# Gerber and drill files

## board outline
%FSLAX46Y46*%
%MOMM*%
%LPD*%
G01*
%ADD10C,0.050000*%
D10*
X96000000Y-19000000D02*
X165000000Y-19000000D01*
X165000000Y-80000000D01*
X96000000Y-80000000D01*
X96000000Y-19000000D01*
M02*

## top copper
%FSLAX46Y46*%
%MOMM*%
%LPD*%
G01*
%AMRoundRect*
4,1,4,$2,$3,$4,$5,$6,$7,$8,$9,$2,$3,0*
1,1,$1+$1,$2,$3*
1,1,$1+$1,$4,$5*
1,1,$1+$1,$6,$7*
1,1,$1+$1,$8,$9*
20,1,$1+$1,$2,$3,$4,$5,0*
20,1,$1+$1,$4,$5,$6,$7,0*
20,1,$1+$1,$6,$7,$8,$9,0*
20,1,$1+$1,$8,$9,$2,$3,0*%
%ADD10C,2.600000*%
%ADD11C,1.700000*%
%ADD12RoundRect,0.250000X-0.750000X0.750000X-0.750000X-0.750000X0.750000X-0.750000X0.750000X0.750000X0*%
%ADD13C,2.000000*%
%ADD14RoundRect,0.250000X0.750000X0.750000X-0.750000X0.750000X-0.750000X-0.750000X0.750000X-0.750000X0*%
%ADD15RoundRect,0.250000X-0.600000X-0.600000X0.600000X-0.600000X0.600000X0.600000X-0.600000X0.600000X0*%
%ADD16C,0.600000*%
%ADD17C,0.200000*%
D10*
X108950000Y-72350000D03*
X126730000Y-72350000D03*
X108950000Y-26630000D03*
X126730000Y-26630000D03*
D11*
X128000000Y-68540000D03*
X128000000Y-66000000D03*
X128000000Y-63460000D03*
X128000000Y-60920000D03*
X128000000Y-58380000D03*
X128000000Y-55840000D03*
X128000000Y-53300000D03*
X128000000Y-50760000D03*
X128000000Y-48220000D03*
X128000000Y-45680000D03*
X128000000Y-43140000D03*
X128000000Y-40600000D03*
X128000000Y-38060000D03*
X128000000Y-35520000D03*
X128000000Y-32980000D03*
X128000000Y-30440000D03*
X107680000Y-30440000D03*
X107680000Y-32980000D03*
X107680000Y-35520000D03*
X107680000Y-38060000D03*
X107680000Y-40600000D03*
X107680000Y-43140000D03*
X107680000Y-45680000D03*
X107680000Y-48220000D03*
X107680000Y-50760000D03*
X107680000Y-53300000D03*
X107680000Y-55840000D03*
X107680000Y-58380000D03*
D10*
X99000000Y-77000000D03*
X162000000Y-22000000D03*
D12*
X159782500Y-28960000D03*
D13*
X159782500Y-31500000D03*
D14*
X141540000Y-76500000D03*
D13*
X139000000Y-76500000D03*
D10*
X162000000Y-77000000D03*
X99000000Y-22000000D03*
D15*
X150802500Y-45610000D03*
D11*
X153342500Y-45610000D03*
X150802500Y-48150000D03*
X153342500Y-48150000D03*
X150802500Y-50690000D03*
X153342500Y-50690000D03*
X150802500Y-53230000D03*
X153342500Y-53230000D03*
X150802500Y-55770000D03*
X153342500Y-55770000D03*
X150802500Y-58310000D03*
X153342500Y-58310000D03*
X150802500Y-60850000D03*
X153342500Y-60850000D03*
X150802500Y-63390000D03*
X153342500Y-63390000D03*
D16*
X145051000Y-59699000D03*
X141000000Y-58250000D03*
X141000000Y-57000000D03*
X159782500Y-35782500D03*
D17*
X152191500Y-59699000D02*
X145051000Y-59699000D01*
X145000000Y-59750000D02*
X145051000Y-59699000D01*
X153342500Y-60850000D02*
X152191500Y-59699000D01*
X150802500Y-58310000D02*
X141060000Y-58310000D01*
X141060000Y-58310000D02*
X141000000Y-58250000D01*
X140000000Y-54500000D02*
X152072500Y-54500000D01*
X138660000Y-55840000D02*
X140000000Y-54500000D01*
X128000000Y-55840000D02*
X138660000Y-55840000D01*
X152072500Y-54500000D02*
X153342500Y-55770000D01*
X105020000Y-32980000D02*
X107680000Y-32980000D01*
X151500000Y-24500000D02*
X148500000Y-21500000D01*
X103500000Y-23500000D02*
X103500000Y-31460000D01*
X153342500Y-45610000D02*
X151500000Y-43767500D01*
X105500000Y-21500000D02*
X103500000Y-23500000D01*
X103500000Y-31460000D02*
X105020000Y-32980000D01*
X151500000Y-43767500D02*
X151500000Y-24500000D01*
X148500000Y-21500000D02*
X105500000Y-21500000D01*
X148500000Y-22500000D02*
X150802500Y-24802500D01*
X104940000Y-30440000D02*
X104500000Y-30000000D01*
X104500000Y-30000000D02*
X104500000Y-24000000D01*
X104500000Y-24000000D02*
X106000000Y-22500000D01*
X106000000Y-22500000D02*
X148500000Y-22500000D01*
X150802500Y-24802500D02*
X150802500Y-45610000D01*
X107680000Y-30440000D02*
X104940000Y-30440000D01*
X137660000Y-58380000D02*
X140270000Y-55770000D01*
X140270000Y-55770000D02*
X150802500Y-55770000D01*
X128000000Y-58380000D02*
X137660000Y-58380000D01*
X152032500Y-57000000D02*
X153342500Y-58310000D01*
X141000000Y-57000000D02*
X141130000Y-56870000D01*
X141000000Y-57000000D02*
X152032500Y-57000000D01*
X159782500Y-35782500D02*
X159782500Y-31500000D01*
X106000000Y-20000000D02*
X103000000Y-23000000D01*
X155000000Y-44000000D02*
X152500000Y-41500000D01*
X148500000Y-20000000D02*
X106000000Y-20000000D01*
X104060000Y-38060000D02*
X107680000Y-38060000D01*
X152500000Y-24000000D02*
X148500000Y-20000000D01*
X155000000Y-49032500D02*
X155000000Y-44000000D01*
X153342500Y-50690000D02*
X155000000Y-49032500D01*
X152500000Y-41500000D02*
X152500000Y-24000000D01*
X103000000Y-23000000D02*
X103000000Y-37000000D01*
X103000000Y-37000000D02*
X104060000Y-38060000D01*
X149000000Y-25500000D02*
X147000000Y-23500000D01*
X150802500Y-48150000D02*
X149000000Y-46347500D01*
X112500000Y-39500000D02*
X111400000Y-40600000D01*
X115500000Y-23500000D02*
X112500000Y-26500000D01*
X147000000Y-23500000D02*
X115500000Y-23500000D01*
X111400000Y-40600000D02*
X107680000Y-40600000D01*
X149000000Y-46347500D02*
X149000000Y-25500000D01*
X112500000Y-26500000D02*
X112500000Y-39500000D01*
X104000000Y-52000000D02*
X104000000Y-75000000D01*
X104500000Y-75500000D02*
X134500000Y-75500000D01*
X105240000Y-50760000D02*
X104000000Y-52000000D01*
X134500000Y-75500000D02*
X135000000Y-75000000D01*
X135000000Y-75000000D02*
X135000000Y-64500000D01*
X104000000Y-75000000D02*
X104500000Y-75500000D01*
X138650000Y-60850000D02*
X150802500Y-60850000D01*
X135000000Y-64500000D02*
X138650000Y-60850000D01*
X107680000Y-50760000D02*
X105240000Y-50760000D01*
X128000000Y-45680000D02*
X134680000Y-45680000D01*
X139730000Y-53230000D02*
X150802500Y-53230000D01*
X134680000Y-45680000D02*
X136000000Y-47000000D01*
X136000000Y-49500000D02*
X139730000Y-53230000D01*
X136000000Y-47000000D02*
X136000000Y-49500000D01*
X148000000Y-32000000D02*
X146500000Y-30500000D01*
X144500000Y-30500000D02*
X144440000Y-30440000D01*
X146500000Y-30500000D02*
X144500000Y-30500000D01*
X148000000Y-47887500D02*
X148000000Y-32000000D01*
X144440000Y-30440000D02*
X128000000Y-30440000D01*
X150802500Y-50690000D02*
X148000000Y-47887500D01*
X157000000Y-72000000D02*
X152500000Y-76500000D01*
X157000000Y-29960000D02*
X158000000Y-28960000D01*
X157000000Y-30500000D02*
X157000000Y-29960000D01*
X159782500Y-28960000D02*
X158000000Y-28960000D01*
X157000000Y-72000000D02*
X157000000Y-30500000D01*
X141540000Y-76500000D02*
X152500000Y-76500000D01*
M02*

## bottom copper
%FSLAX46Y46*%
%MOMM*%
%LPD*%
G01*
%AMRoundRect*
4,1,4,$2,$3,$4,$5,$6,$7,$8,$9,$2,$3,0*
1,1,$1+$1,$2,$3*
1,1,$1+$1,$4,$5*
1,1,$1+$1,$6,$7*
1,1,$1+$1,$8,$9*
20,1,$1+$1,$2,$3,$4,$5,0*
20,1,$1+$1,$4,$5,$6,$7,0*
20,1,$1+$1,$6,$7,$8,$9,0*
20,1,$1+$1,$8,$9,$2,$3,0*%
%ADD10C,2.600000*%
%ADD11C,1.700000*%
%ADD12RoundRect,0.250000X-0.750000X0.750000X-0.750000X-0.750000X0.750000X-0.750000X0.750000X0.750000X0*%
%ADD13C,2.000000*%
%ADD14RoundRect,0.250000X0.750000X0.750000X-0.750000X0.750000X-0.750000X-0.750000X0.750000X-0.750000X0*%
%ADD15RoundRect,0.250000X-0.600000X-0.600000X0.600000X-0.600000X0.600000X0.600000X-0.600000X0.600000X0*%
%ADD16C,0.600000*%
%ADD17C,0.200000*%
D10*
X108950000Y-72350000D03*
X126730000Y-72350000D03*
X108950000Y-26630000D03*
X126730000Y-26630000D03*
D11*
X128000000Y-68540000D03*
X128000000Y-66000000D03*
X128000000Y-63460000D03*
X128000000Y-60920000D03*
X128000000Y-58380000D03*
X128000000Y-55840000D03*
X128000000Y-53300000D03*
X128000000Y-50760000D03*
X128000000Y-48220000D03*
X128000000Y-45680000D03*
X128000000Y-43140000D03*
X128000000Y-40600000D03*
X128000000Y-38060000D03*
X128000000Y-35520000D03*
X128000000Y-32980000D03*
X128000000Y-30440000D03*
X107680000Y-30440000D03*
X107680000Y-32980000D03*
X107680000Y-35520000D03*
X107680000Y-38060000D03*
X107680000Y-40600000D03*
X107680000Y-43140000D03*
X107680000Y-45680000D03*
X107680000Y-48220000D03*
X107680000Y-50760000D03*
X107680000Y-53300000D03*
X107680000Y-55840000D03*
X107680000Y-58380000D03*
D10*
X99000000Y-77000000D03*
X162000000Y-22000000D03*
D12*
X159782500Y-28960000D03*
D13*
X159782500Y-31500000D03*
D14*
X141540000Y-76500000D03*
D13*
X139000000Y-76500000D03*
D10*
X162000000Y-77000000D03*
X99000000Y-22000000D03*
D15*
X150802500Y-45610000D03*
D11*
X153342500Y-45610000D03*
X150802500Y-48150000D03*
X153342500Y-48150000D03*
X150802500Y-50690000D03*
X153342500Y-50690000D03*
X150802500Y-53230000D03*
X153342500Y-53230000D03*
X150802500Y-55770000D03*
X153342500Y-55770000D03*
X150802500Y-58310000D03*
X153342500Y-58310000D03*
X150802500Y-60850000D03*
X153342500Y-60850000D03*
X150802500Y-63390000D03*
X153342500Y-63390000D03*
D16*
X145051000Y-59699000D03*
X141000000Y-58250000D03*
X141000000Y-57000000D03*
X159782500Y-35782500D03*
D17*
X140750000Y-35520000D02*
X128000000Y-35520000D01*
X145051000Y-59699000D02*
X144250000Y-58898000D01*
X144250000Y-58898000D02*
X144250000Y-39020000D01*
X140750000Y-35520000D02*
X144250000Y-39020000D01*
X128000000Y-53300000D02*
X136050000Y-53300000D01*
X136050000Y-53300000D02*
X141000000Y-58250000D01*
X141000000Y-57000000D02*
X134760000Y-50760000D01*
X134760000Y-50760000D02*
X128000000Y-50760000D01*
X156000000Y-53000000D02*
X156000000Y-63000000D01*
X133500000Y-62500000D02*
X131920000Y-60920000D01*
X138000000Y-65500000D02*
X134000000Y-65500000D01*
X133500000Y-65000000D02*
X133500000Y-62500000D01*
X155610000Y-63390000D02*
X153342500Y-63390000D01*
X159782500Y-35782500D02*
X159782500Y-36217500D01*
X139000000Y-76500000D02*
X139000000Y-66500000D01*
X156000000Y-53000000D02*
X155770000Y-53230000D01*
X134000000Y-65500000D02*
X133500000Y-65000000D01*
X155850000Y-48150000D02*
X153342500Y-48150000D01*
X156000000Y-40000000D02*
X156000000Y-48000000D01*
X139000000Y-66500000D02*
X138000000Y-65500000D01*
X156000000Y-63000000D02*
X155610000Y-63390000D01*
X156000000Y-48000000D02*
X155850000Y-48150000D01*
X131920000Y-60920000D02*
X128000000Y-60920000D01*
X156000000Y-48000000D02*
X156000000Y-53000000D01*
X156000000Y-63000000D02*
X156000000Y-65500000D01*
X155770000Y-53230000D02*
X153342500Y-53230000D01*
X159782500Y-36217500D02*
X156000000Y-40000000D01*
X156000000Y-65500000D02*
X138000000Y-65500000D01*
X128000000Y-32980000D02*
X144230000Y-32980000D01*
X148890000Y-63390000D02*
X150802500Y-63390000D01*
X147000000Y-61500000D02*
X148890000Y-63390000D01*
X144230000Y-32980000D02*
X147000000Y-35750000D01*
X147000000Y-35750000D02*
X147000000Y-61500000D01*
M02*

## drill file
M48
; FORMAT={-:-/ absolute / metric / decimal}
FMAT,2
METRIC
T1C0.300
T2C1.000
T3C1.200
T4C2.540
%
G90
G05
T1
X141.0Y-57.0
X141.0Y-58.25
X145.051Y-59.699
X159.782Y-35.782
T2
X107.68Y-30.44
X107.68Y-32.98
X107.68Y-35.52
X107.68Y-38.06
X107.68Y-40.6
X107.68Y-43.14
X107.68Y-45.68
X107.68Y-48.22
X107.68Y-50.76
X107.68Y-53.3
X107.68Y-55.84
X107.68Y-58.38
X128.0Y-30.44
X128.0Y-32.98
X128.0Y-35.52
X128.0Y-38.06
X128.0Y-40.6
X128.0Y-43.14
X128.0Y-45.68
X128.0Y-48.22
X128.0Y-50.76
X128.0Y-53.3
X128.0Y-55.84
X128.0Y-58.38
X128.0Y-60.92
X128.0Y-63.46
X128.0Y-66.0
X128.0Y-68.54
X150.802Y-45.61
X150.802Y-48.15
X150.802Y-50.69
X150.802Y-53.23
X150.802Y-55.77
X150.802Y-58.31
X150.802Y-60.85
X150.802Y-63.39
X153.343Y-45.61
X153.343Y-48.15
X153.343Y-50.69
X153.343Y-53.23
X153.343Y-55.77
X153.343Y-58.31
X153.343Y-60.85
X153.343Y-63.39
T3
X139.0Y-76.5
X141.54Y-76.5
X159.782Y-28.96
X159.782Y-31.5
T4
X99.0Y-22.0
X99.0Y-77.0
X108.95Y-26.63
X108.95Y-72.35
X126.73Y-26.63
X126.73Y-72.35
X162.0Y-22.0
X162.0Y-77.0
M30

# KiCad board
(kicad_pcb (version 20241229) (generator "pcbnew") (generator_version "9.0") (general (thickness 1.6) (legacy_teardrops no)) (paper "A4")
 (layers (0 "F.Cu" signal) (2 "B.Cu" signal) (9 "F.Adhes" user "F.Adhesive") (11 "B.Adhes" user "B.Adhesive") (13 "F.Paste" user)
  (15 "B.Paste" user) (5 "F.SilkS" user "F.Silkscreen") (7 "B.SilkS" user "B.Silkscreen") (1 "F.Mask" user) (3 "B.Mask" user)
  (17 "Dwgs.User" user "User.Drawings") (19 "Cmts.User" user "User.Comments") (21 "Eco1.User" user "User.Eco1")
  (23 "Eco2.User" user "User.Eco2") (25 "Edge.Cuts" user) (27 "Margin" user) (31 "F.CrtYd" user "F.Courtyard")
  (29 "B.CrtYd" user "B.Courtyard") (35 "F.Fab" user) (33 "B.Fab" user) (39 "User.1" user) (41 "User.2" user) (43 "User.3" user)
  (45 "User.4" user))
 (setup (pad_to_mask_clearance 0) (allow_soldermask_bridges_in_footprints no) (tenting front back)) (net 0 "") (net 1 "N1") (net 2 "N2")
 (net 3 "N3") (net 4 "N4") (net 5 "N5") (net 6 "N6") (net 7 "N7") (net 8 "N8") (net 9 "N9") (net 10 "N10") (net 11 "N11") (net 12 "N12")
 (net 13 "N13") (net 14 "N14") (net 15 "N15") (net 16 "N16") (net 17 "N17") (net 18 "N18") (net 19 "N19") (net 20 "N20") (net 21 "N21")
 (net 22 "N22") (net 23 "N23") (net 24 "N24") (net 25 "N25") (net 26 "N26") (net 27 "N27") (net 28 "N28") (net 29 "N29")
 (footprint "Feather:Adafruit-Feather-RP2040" (layer "F.Cu") (at 117.84 49.49 90)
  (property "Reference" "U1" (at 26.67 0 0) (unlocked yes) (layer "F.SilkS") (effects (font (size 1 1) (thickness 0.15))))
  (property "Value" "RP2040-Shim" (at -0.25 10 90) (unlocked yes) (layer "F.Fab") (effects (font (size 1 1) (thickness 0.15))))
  (pad "" np_thru_hole circle (at -22.86 -8.89 90) (size 2.6 2.6) (drill 2.54) (layers "*.Cu" "*.Mask") (solder_mask_margin 1.3)
   (clearance 1.3))
  (pad "" np_thru_hole circle (at -22.86 8.89 90) (size 2.6 2.6) (drill 2.54) (layers "*.Cu" "*.Mask") (solder_mask_margin 1.3)
   (clearance 1.3))
  (pad "" np_thru_hole circle (at 22.86 -8.89 90) (size 2.6 2.6) (drill 2.54) (layers "*.Cu" "*.Mask") (solder_mask_margin 1.3)
   (clearance 1.3))
  (pad "" np_thru_hole circle (at 22.86 8.89 90) (size 2.6 2.6) (drill 2.54) (layers "*.Cu" "*.Mask") (solder_mask_margin 1.3)
   (clearance 1.3))
  (pad "1" thru_hole circle (at -19.05 10.16 90) (size 1.7 1.7) (drill 1) (layers "*.Cu" "*.Mask") (remove_unused_layers no) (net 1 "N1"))
  (pad "2" thru_hole circle (at -16.51 10.16 90) (size 1.7 1.7) (drill 1) (layers "*.Cu" "*.Mask") (remove_unused_layers no) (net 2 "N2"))
  (pad "3" thru_hole circle (at -13.97 10.16 90) (size 1.7 1.7) (drill 1) (layers "*.Cu" "*.Mask") (remove_unused_layers no) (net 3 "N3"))
  (pad "4" thru_hole circle (at -11.43 10.16 90) (size 1.7 1.7) (drill 1) (layers "*.Cu" "*.Mask") (remove_unused_layers no) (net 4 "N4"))
  (pad "5" thru_hole circle (at -8.89 10.16 90) (size 1.7 1.7) (drill 1) (layers "*.Cu" "*.Mask") (remove_unused_layers no) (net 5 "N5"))
  (pad "6" thru_hole circle (at -6.35 10.16 90) (size 1.7 1.7) (drill 1) (layers "*.Cu" "*.Mask") (remove_unused_layers no) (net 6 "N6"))
  (pad "7" thru_hole circle (at -3.81 10.16 90) (size 1.7 1.7) (drill 1) (layers "*.Cu" "*.Mask") (remove_unused_layers no) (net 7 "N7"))
  (pad "8" thru_hole circle (at -1.27 10.16 90) (size 1.7 1.7) (drill 1) (layers "*.Cu" "*.Mask") (remove_unused_layers no) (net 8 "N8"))
  (pad "9" thru_hole circle (at 1.27 10.16 90) (size 1.7 1.7) (drill 1) (layers "*.Cu" "*.Mask") (remove_unused_layers no) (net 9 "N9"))
  (pad "10" thru_hole circle (at 3.81 10.16 90) (size 1.7 1.7) (drill 1) (layers "*.Cu" "*.Mask") (remove_unused_layers no) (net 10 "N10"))
  (pad "11" thru_hole circle (at 6.35 10.16 90) (size 1.7 1.7) (drill 1) (layers "*.Cu" "*.Mask") (remove_unused_layers no) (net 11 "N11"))
  (pad "12" thru_hole circle (at 8.89 10.16 90) (size 1.7 1.7) (drill 1) (layers "*.Cu" "*.Mask") (remove_unused_layers no) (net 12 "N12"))
  (pad "13" thru_hole circle (at 11.43 10.16 90) (size 1.7 1.7) (drill 1) (layers "*.Cu" "*.Mask") (remove_unused_layers no) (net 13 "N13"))
  (pad "14" thru_hole circle (at 13.97 10.16 90) (size 1.7 1.7) (drill 1) (layers "*.Cu" "*.Mask") (remove_unused_layers no) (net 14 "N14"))
  (pad "15" thru_hole circle (at 16.51 10.16 90) (size 1.7 1.7) (drill 1) (layers "*.Cu" "*.Mask") (remove_unused_layers no) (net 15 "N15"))
  (pad "16" thru_hole circle (at 19.05 10.16 90) (size 1.7 1.7) (drill 1) (layers "*.Cu" "*.Mask") (remove_unused_layers no) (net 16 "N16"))
  (pad "17" thru_hole circle (at 19.05 -10.16 90) (size 1.7 1.7) (drill 1) (layers "*.Cu" "*.Mask") (remove_unused_layers no) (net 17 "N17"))
  (pad "18" thru_hole circle (at 16.51 -10.16 90) (size 1.7 1.7) (drill 1) (layers "*.Cu" "*.Mask") (remove_unused_layers no) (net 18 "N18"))
  (pad "19" thru_hole circle (at 13.97 -10.16 90) (size 1.7 1.7) (drill 1) (layers "*.Cu" "*.Mask") (remove_unused_layers no) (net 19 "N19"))
  (pad "20" thru_hole circle (at 11.43 -10.16 90) (size 1.7 1.7) (drill 1) (layers "*.Cu" "*.Mask") (remove_unused_layers no) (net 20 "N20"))
  (pad "21" thru_hole circle (at 8.89 -10.16 90) (size 1.7 1.7) (drill 1) (layers "*.Cu" "*.Mask") (remove_unused_layers no) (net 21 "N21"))
  (pad "22" thru_hole circle (at 6.35 -10.16 90) (size 1.7 1.7) (drill 1) (layers "*.Cu" "*.Mask") (remove_unused_layers no) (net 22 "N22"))
  (pad "23" thru_hole circle (at 3.81 -10.16 90) (size 1.7 1.7) (drill 1) (layers "*.Cu" "*.Mask") (remove_unused_layers no) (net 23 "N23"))
  (pad "24" thru_hole circle (at 1.27 -10.16 90) (size 1.7 1.7) (drill 1) (layers "*.Cu" "*.Mask") (remove_unused_layers no) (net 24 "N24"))
  (pad "25" thru_hole circle (at -1.27 -10.16 90) (size 1.7 1.7) (drill 1) (layers "*.Cu" "*.Mask") (remove_unused_layers no) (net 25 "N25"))
  (pad "26" thru_hole circle (at -3.81 -10.16 90) (size 1.7 1.7) (drill 1) (layers "*.Cu" "*.Mask") (remove_unused_layers no) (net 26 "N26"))
  (pad "27" thru_hole circle (at -6.35 -10.16 90) (size 1.7 1.7) (drill 1) (layers "*.Cu" "*.Mask") (remove_unused_layers no) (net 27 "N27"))
  (pad "28" thru_hole circle (at -8.89 -10.16 90) (size 1.7 1.7) (drill 1) (layers "*.Cu" "*.Mask") (remove_unused_layers no) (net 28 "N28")))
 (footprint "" (layer "F.Cu") (at 99 77)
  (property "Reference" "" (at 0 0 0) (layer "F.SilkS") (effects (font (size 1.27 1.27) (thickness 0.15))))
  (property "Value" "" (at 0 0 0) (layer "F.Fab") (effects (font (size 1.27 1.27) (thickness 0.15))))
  (pad "" np_thru_hole circle (at 0 0 90) (size 2.6 2.6) (drill 2.54) (layers "*.Cu" "*.Mask") (solder_mask_margin 1.3) (clearance 1.3)))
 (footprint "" (layer "F.Cu") (at 162 22)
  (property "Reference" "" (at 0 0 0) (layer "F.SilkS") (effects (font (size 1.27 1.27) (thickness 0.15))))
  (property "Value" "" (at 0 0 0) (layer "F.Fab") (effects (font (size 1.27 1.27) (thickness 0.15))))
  (pad "" np_thru_hole circle (at 0 0 90) (size 2.6 2.6) (drill 2.54) (layers "*.Cu" "*.Mask") (solder_mask_margin 1.3) (clearance 1.3)))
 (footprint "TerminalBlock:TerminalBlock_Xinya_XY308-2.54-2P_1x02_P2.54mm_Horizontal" (layer "F.Cu") (at 159.7825 28.96 -90)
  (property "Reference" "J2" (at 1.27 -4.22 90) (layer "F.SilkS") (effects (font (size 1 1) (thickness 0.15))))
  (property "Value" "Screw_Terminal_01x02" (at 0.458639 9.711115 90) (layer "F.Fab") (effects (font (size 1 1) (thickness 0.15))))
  (pad "1" thru_hole roundrect (at 0 0 270) (size 2 2) (drill 1.2) (layers "*.Cu" "*.Mask") (remove_unused_layers no)
   (roundrect_rratio 0.125) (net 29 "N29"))
  (pad "2" thru_hole circle (at 2.54 0 270) (size 2 2) (drill 1.2) (layers "*.Cu" "*.Mask") (remove_unused_layers no) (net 4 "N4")))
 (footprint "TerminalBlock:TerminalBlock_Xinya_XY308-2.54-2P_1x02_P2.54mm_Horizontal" (layer "F.Cu") (at 141.54 76.5 180)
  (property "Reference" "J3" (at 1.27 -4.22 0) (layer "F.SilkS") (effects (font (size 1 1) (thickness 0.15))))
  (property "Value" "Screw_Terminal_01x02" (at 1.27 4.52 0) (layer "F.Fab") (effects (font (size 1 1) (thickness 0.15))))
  (pad "1" thru_hole roundrect (at 0 0 180) (size 2 2) (drill 1.2) (layers "*.Cu" "*.Mask") (remove_unused_layers no)
   (roundrect_rratio 0.125) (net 29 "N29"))
  (pad "2" thru_hole circle (at 2.54 0 180) (size 2 2) (drill 1.2) (layers "*.Cu" "*.Mask") (remove_unused_layers no) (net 4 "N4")))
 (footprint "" (layer "F.Cu") (at 162 77)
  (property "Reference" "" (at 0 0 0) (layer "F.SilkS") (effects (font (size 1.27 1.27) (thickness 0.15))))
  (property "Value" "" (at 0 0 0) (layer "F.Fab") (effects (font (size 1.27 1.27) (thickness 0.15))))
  (pad "" np_thru_hole circle (at 0 0 90) (size 2.6 2.6) (drill 2.54) (layers "*.Cu" "*.Mask") (solder_mask_margin 1.3) (clearance 1.3)))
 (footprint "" (layer "F.Cu") (at 99 22)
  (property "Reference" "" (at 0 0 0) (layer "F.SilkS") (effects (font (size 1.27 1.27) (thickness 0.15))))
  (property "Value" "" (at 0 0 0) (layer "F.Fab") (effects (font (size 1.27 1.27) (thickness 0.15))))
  (pad "" np_thru_hole circle (at 0 0 90) (size 2.6 2.6) (drill 2.54) (layers "*.Cu" "*.Mask") (solder_mask_margin 1.3) (clearance 1.3)))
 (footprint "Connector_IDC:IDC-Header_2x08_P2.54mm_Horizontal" (layer "F.Cu") (at 150.8025 45.61)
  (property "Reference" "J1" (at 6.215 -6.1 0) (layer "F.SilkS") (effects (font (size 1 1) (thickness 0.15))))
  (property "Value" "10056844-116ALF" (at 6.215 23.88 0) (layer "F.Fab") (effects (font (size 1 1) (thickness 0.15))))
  (pad "1" thru_hole roundrect (at 0 0) (size 1.7 1.7) (drill 1) (layers "*.Cu" "*.Mask") (remove_unused_layers no)
   (roundrect_rratio 0.147059) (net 17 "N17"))
  (pad "2" thru_hole circle (at 2.54 0) (size 1.7 1.7) (drill 1) (layers "*.Cu" "*.Mask") (remove_unused_layers no) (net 18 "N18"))
  (pad "3" thru_hole circle (at 0 2.54) (size 1.7 1.7) (drill 1) (layers "*.Cu" "*.Mask") (remove_unused_layers no) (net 21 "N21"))
  (pad "4" thru_hole circle (at 2.54 2.54) (size 1.7 1.7) (drill 1) (layers "*.Cu" "*.Mask") (remove_unused_layers no) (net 4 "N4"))
  (pad "5" thru_hole circle (at 0 5.08) (size 1.7 1.7) (drill 1) (layers "*.Cu" "*.Mask") (remove_unused_layers no) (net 16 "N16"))
  (pad "6" thru_hole circle (at 2.54 5.08) (size 1.7 1.7) (drill 1) (layers "*.Cu" "*.Mask") (remove_unused_layers no) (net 20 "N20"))
  (pad "7" thru_hole circle (at 0 7.62) (size 1.7 1.7) (drill 1) (layers "*.Cu" "*.Mask") (remove_unused_layers no) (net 10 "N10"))
  (pad "8" thru_hole circle (at 2.54 7.62) (size 1.7 1.7) (drill 1) (layers "*.Cu" "*.Mask") (remove_unused_layers no) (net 4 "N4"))
  (pad "9" thru_hole circle (at 0 10.16) (size 1.7 1.7) (drill 1) (layers "*.Cu" "*.Mask") (remove_unused_layers no) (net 5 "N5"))
  (pad "10" thru_hole circle (at 2.54 10.16) (size 1.7 1.7) (drill 1) (layers "*.Cu" "*.Mask") (remove_unused_layers no) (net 6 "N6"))
  (pad "11" thru_hole circle (at 0 12.7) (size 1.7 1.7) (drill 1) (layers "*.Cu" "*.Mask") (remove_unused_layers no) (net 7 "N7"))
  (pad "12" thru_hole circle (at 2.54 12.7) (size 1.7 1.7) (drill 1) (layers "*.Cu" "*.Mask") (remove_unused_layers no) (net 8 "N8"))
  (pad "13" thru_hole circle (at 0 15.24) (size 1.7 1.7) (drill 1) (layers "*.Cu" "*.Mask") (remove_unused_layers no) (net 25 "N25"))
  (pad "14" thru_hole circle (at 2.54 15.24) (size 1.7 1.7) (drill 1) (layers "*.Cu" "*.Mask") (remove_unused_layers no) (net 14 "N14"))
  (pad "15" thru_hole circle (at 0 17.78) (size 1.7 1.7) (drill 1) (layers "*.Cu" "*.Mask") (remove_unused_layers no) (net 15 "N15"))
  (pad "16" thru_hole circle (at 2.54 17.78) (size 1.7 1.7) (drill 1) (layers "*.Cu" "*.Mask") (remove_unused_layers no) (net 4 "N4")))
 (gr_rect (start 96 19) (end 165 80) (stroke (width 0.05) (type solid)) (fill no) (layer "Edge.Cuts"))
 (segment (start 152.1915 59.699) (end 145.051 59.699) (width 0.2) (layer "F.Cu") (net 14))
 (segment (start 145 59.75) (end 145.051 59.699) (width 0.2) (layer "F.Cu") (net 14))
 (segment (start 153.3425 60.85) (end 152.1915 59.699) (width 0.2) (layer "F.Cu") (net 14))
 (via (at 145.051 59.699) (size 0.6) (drill 0.3) (layers "F.Cu" "B.Cu") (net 14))
 (segment (start 140.75 35.52) (end 128 35.52) (width 0.2) (layer "B.Cu") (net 14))
 (segment (start 145.051 59.699) (end 144.25 58.898) (width 0.2) (layer "B.Cu") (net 14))
 (segment (start 144.25 58.898) (end 144.25 39.02) (width 0.2) (layer "B.Cu") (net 14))
 (segment (start 140.75 35.52) (end 144.25 39.02) (width 0.2) (layer "B.Cu") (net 14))
 (segment (start 150.8025 58.31) (end 141.06 58.31) (width 0.2) (layer "F.Cu") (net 7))
 (segment (start 141.06 58.31) (end 141 58.25) (width 0.2) (layer "F.Cu") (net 7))
 (via (at 141 58.25) (size 0.6) (drill 0.3) (layers "F.Cu" "B.Cu") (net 7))
 (segment (start 128 53.3) (end 136.05 53.3) (width 0.2) (layer "B.Cu") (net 7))
 (segment (start 136.05 53.3) (end 141 58.25) (width 0.2) (layer "B.Cu") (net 7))
 (segment (start 140 54.5) (end 152.0725 54.5) (width 0.2) (layer "F.Cu") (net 6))
 (segment (start 138.66 55.84) (end 140 54.5) (width 0.2) (layer "F.Cu") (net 6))
 (segment (start 128 55.84) (end 138.66 55.84) (width 0.2) (layer "F.Cu") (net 6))
 (segment (start 152.0725 54.5) (end 153.3425 55.77) (width 0.2) (layer "F.Cu") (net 6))
 (segment (start 105.02 32.98) (end 107.68 32.98) (width 0.2) (layer "F.Cu") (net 18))
 (segment (start 151.5 24.5) (end 148.5 21.5) (width 0.2) (layer "F.Cu") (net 18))
 (segment (start 103.5 23.5) (end 103.5 31.46) (width 0.2) (layer "F.Cu") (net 18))
 (segment (start 153.3425 45.61) (end 151.5 43.7675) (width 0.2) (layer "F.Cu") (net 18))
 (segment (start 105.5 21.5) (end 103.5 23.5) (width 0.2) (layer "F.Cu") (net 18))
 (segment (start 103.5 31.46) (end 105.02 32.98) (width 0.2) (layer "F.Cu") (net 18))
 (segment (start 151.5 43.7675) (end 151.5 24.5) (width 0.2) (layer "F.Cu") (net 18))
 (segment (start 148.5 21.5) (end 105.5 21.5) (width 0.2) (layer "F.Cu") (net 18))
 (segment (start 148.5 22.5) (end 150.8025 24.8025) (width 0.2) (layer "F.Cu") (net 17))
 (segment (start 104.94 30.44) (end 104.5 30) (width 0.2) (layer "F.Cu") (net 17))
 (segment (start 104.5 30) (end 104.5 24) (width 0.2) (layer "F.Cu") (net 17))
 (segment (start 104.5 24) (end 106 22.5) (width 0.2) (layer "F.Cu") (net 17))
 (segment (start 106 22.5) (end 148.5 22.5) (width 0.2) (layer "F.Cu") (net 17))
 (segment (start 150.8025 24.8025) (end 150.8025 45.61) (width 0.2) (layer "F.Cu") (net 17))
 (segment (start 107.68 30.44) (end 104.94 30.44) (width 0.2) (layer "F.Cu") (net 17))
 (segment (start 137.66 58.38) (end 140.27 55.77) (width 0.2) (layer "F.Cu") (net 5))
 (segment (start 140.27 55.77) (end 150.8025 55.77) (width 0.2) (layer "F.Cu") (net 5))
 (segment (start 128 58.38) (end 137.66 58.38) (width 0.2) (layer "F.Cu") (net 5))
 (segment (start 152.0325 57) (end 153.3425 58.31) (width 0.2) (layer "F.Cu") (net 8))
 (segment (start 141 57) (end 141.13 56.87) (width 0.2) (layer "F.Cu") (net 8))
 (segment (start 141 57) (end 152.0325 57) (width 0.2) (layer "F.Cu") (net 8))
 (via (at 141 57) (size 0.6) (drill 0.3) (layers "F.Cu" "B.Cu") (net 8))
 (segment (start 141 57) (end 134.76 50.76) (width 0.2) (layer "B.Cu") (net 8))
 (segment (start 134.76 50.76) (end 128 50.76) (width 0.2) (layer "B.Cu") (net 8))
 (segment (start 159.7825 35.7825) (end 159.7825 31.5) (width 0.2) (layer "F.Cu") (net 4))
 (via (at 159.7825 35.7825) (size 0.6) (drill 0.3) (layers "F.Cu" "B.Cu") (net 4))
 (segment (start 156 53) (end 156 63) (width 0.2) (layer "B.Cu") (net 4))
 (segment (start 133.5 62.5) (end 131.92 60.92) (width 0.2) (layer "B.Cu") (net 4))
 (segment (start 138 65.5) (end 134 65.5) (width 0.2) (layer "B.Cu") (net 4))
 (segment (start 133.5 65) (end 133.5 62.5) (width 0.2) (layer "B.Cu") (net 4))
 (segment (start 155.61 63.39) (end 153.3425 63.39) (width 0.2) (layer "B.Cu") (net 4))
 (segment (start 159.7825 35.7825) (end 159.7825 36.2175) (width 0.2) (layer "B.Cu") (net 4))
 (segment (start 139 76.5) (end 139 66.5) (width 0.2) (layer "B.Cu") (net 4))
 (segment (start 156 53) (end 155.77 53.23) (width 0.2) (layer "B.Cu") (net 4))
 (segment (start 134 65.5) (end 133.5 65) (width 0.2) (layer "B.Cu") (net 4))
 (segment (start 155.85 48.15) (end 153.3425 48.15) (width 0.2) (layer "B.Cu") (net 4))
 (segment (start 156 40) (end 156 48) (width 0.2) (layer "B.Cu") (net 4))
 (segment (start 139 66.5) (end 138 65.5) (width 0.2) (layer "B.Cu") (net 4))
 (segment (start 156 63) (end 155.61 63.39) (width 0.2) (layer "B.Cu") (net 4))
 (segment (start 156 48) (end 155.85 48.15) (width 0.2) (layer "B.Cu") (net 4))
 (segment (start 131.92 60.92) (end 128 60.92) (width 0.2) (layer "B.Cu") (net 4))
 (segment (start 156 48) (end 156 53) (width 0.2) (layer "B.Cu") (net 4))
 (segment (start 156 63) (end 156 65.5) (width 0.2) (layer "B.Cu") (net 4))
 (segment (start 155.77 53.23) (end 153.3425 53.23) (width 0.2) (layer "B.Cu") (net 4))
 (segment (start 159.7825 36.2175) (end 156 40) (width 0.2) (layer "B.Cu") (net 4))
 (segment (start 156 65.5) (end 138 65.5) (width 0.2) (layer "B.Cu") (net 4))
 (segment (start 128 32.98) (end 144.23 32.98) (width 0.2) (layer "B.Cu") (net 15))
 (segment (start 148.89 63.39) (end 150.8025 63.39) (width 0.2) (layer "B.Cu") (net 15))
 (segment (start 147 61.5) (end 148.89 63.39) (width 0.2) (layer "B.Cu") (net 15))
 (segment (start 144.23 32.98) (end 147 35.75) (width 0.2) (layer "B.Cu") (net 15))
 (segment (start 147 35.75) (end 147 61.5) (width 0.2) (layer "B.Cu") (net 15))
 (segment (start 106 20) (end 103 23) (width 0.2) (layer "F.Cu") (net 20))
 (segment (start 155 44) (end 152.5 41.5) (width 0.2) (layer "F.Cu") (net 20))
 (segment (start 148.5 20) (end 106 20) (width 0.2) (layer "F.Cu") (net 20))
 (segment (start 104.06 38.06) (end 107.68 38.06) (width 0.2) (layer "F.Cu") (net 20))
 (segment (start 152.5 24) (end 148.5 20) (width 0.2) (layer "F.Cu") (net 20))
 (segment (start 155 49.0325) (end 155 44) (width 0.2) (layer "F.Cu") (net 20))
 (segment (start 153.3425 50.69) (end 155 49.0325) (width 0.2) (layer "F.Cu") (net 20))
 (segment (start 152.5 41.5) (end 152.5 24) (width 0.2) (layer "F.Cu") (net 20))
 (segment (start 103 23) (end 103 37) (width 0.2) (layer "F.Cu") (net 20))
 (segment (start 103 37) (end 104.06 38.06) (width 0.2) (layer "F.Cu") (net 20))
 (segment (start 149 25.5) (end 147 23.5) (width 0.2) (layer "F.Cu") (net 21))
 (segment (start 150.8025 48.15) (end 149 46.3475) (width 0.2) (layer "F.Cu") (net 21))
 (segment (start 112.5 39.5) (end 111.4 40.6) (width 0.2) (layer "F.Cu") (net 21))
 (segment (start 115.5 23.5) (end 112.5 26.5) (width 0.2) (layer "F.Cu") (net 21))
 (segment (start 147 23.5) (end 115.5 23.5) (width 0.2) (layer "F.Cu") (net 21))
 (segment (start 111.4 40.6) (end 107.68 40.6) (width 0.2) (layer "F.Cu") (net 21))
 (segment (start 149 46.3475) (end 149 25.5) (width 0.2) (layer "F.Cu") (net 21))
 (segment (start 112.5 26.5) (end 112.5 39.5) (width 0.2) (layer "F.Cu") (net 21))
 (segment (start 104 52) (end 104 75) (width 0.2) (layer "F.Cu") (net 25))
 (segment (start 104.5 75.5) (end 134.5 75.5) (width 0.2) (layer "F.Cu") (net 25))
 (segment (start 105.24 50.76) (end 104 52) (width 0.2) (layer "F.Cu") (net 25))
 (segment (start 134.5 75.5) (end 135 75) (width 0.2) (layer "F.Cu") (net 25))
 (segment (start 135 75) (end 135 64.5) (width 0.2) (layer "F.Cu") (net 25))
 (segment (start 104 75) (end 104.5 75.5) (width 0.2) (layer "F.Cu") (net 25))
 (segment (start 138.65 60.85) (end 150.8025 60.85) (width 0.2) (layer "F.Cu") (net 25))
 (segment (start 135 64.5) (end 138.65 60.85) (width 0.2) (layer "F.Cu") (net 25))
 (segment (start 107.68 50.76) (end 105.24 50.76) (width 0.2) (layer "F.Cu") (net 25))
 (segment (start 128 45.68) (end 134.68 45.68) (width 0.2) (layer "F.Cu") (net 10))
 (segment (start 139.73 53.23) (end 150.8025 53.23) (width 0.2) (layer "F.Cu") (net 10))
 (segment (start 134.68 45.68) (end 136 47) (width 0.2) (layer "F.Cu") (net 10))
 (segment (start 136 49.5) (end 139.73 53.23) (width 0.2) (layer "F.Cu") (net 10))
 (segment (start 136 47) (end 136 49.5) (width 0.2) (layer "F.Cu") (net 10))
 (segment (start 148 32) (end 146.5 30.5) (width 0.2) (layer "F.Cu") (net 16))
 (segment (start 144.5 30.5) (end 144.44 30.44) (width 0.2) (layer "F.Cu") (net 16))
 (segment (start 146.5 30.5) (end 144.5 30.5) (width 0.2) (layer "F.Cu") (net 16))
 (segment (start 148 47.8875) (end 148 32) (width 0.2) (layer "F.Cu") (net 16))
 (segment (start 144.44 30.44) (end 128 30.44) (width 0.2) (layer "F.Cu") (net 16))
 (segment (start 150.8025 50.69) (end 148 47.8875) (width 0.2) (layer "F.Cu") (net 16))
 (segment (start 157 72) (end 152.5 76.5) (width 0.2) (layer "F.Cu") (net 29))
 (segment (start 157 29.96) (end 158 28.96) (width 0.2) (layer "F.Cu") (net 29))
 (segment (start 157 30.5) (end 157 29.96) (width 0.2) (layer "F.Cu") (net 29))
 (segment (start 159.7825 28.96) (end 158 28.96) (width 0.2) (layer "F.Cu") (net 29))
 (segment (start 157 72) (end 157 30.5) (width 0.2) (layer "F.Cu") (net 29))
 (segment (start 141.54 76.5) (end 152.5 76.5) (width 0.2) (layer "F.Cu") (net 29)))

